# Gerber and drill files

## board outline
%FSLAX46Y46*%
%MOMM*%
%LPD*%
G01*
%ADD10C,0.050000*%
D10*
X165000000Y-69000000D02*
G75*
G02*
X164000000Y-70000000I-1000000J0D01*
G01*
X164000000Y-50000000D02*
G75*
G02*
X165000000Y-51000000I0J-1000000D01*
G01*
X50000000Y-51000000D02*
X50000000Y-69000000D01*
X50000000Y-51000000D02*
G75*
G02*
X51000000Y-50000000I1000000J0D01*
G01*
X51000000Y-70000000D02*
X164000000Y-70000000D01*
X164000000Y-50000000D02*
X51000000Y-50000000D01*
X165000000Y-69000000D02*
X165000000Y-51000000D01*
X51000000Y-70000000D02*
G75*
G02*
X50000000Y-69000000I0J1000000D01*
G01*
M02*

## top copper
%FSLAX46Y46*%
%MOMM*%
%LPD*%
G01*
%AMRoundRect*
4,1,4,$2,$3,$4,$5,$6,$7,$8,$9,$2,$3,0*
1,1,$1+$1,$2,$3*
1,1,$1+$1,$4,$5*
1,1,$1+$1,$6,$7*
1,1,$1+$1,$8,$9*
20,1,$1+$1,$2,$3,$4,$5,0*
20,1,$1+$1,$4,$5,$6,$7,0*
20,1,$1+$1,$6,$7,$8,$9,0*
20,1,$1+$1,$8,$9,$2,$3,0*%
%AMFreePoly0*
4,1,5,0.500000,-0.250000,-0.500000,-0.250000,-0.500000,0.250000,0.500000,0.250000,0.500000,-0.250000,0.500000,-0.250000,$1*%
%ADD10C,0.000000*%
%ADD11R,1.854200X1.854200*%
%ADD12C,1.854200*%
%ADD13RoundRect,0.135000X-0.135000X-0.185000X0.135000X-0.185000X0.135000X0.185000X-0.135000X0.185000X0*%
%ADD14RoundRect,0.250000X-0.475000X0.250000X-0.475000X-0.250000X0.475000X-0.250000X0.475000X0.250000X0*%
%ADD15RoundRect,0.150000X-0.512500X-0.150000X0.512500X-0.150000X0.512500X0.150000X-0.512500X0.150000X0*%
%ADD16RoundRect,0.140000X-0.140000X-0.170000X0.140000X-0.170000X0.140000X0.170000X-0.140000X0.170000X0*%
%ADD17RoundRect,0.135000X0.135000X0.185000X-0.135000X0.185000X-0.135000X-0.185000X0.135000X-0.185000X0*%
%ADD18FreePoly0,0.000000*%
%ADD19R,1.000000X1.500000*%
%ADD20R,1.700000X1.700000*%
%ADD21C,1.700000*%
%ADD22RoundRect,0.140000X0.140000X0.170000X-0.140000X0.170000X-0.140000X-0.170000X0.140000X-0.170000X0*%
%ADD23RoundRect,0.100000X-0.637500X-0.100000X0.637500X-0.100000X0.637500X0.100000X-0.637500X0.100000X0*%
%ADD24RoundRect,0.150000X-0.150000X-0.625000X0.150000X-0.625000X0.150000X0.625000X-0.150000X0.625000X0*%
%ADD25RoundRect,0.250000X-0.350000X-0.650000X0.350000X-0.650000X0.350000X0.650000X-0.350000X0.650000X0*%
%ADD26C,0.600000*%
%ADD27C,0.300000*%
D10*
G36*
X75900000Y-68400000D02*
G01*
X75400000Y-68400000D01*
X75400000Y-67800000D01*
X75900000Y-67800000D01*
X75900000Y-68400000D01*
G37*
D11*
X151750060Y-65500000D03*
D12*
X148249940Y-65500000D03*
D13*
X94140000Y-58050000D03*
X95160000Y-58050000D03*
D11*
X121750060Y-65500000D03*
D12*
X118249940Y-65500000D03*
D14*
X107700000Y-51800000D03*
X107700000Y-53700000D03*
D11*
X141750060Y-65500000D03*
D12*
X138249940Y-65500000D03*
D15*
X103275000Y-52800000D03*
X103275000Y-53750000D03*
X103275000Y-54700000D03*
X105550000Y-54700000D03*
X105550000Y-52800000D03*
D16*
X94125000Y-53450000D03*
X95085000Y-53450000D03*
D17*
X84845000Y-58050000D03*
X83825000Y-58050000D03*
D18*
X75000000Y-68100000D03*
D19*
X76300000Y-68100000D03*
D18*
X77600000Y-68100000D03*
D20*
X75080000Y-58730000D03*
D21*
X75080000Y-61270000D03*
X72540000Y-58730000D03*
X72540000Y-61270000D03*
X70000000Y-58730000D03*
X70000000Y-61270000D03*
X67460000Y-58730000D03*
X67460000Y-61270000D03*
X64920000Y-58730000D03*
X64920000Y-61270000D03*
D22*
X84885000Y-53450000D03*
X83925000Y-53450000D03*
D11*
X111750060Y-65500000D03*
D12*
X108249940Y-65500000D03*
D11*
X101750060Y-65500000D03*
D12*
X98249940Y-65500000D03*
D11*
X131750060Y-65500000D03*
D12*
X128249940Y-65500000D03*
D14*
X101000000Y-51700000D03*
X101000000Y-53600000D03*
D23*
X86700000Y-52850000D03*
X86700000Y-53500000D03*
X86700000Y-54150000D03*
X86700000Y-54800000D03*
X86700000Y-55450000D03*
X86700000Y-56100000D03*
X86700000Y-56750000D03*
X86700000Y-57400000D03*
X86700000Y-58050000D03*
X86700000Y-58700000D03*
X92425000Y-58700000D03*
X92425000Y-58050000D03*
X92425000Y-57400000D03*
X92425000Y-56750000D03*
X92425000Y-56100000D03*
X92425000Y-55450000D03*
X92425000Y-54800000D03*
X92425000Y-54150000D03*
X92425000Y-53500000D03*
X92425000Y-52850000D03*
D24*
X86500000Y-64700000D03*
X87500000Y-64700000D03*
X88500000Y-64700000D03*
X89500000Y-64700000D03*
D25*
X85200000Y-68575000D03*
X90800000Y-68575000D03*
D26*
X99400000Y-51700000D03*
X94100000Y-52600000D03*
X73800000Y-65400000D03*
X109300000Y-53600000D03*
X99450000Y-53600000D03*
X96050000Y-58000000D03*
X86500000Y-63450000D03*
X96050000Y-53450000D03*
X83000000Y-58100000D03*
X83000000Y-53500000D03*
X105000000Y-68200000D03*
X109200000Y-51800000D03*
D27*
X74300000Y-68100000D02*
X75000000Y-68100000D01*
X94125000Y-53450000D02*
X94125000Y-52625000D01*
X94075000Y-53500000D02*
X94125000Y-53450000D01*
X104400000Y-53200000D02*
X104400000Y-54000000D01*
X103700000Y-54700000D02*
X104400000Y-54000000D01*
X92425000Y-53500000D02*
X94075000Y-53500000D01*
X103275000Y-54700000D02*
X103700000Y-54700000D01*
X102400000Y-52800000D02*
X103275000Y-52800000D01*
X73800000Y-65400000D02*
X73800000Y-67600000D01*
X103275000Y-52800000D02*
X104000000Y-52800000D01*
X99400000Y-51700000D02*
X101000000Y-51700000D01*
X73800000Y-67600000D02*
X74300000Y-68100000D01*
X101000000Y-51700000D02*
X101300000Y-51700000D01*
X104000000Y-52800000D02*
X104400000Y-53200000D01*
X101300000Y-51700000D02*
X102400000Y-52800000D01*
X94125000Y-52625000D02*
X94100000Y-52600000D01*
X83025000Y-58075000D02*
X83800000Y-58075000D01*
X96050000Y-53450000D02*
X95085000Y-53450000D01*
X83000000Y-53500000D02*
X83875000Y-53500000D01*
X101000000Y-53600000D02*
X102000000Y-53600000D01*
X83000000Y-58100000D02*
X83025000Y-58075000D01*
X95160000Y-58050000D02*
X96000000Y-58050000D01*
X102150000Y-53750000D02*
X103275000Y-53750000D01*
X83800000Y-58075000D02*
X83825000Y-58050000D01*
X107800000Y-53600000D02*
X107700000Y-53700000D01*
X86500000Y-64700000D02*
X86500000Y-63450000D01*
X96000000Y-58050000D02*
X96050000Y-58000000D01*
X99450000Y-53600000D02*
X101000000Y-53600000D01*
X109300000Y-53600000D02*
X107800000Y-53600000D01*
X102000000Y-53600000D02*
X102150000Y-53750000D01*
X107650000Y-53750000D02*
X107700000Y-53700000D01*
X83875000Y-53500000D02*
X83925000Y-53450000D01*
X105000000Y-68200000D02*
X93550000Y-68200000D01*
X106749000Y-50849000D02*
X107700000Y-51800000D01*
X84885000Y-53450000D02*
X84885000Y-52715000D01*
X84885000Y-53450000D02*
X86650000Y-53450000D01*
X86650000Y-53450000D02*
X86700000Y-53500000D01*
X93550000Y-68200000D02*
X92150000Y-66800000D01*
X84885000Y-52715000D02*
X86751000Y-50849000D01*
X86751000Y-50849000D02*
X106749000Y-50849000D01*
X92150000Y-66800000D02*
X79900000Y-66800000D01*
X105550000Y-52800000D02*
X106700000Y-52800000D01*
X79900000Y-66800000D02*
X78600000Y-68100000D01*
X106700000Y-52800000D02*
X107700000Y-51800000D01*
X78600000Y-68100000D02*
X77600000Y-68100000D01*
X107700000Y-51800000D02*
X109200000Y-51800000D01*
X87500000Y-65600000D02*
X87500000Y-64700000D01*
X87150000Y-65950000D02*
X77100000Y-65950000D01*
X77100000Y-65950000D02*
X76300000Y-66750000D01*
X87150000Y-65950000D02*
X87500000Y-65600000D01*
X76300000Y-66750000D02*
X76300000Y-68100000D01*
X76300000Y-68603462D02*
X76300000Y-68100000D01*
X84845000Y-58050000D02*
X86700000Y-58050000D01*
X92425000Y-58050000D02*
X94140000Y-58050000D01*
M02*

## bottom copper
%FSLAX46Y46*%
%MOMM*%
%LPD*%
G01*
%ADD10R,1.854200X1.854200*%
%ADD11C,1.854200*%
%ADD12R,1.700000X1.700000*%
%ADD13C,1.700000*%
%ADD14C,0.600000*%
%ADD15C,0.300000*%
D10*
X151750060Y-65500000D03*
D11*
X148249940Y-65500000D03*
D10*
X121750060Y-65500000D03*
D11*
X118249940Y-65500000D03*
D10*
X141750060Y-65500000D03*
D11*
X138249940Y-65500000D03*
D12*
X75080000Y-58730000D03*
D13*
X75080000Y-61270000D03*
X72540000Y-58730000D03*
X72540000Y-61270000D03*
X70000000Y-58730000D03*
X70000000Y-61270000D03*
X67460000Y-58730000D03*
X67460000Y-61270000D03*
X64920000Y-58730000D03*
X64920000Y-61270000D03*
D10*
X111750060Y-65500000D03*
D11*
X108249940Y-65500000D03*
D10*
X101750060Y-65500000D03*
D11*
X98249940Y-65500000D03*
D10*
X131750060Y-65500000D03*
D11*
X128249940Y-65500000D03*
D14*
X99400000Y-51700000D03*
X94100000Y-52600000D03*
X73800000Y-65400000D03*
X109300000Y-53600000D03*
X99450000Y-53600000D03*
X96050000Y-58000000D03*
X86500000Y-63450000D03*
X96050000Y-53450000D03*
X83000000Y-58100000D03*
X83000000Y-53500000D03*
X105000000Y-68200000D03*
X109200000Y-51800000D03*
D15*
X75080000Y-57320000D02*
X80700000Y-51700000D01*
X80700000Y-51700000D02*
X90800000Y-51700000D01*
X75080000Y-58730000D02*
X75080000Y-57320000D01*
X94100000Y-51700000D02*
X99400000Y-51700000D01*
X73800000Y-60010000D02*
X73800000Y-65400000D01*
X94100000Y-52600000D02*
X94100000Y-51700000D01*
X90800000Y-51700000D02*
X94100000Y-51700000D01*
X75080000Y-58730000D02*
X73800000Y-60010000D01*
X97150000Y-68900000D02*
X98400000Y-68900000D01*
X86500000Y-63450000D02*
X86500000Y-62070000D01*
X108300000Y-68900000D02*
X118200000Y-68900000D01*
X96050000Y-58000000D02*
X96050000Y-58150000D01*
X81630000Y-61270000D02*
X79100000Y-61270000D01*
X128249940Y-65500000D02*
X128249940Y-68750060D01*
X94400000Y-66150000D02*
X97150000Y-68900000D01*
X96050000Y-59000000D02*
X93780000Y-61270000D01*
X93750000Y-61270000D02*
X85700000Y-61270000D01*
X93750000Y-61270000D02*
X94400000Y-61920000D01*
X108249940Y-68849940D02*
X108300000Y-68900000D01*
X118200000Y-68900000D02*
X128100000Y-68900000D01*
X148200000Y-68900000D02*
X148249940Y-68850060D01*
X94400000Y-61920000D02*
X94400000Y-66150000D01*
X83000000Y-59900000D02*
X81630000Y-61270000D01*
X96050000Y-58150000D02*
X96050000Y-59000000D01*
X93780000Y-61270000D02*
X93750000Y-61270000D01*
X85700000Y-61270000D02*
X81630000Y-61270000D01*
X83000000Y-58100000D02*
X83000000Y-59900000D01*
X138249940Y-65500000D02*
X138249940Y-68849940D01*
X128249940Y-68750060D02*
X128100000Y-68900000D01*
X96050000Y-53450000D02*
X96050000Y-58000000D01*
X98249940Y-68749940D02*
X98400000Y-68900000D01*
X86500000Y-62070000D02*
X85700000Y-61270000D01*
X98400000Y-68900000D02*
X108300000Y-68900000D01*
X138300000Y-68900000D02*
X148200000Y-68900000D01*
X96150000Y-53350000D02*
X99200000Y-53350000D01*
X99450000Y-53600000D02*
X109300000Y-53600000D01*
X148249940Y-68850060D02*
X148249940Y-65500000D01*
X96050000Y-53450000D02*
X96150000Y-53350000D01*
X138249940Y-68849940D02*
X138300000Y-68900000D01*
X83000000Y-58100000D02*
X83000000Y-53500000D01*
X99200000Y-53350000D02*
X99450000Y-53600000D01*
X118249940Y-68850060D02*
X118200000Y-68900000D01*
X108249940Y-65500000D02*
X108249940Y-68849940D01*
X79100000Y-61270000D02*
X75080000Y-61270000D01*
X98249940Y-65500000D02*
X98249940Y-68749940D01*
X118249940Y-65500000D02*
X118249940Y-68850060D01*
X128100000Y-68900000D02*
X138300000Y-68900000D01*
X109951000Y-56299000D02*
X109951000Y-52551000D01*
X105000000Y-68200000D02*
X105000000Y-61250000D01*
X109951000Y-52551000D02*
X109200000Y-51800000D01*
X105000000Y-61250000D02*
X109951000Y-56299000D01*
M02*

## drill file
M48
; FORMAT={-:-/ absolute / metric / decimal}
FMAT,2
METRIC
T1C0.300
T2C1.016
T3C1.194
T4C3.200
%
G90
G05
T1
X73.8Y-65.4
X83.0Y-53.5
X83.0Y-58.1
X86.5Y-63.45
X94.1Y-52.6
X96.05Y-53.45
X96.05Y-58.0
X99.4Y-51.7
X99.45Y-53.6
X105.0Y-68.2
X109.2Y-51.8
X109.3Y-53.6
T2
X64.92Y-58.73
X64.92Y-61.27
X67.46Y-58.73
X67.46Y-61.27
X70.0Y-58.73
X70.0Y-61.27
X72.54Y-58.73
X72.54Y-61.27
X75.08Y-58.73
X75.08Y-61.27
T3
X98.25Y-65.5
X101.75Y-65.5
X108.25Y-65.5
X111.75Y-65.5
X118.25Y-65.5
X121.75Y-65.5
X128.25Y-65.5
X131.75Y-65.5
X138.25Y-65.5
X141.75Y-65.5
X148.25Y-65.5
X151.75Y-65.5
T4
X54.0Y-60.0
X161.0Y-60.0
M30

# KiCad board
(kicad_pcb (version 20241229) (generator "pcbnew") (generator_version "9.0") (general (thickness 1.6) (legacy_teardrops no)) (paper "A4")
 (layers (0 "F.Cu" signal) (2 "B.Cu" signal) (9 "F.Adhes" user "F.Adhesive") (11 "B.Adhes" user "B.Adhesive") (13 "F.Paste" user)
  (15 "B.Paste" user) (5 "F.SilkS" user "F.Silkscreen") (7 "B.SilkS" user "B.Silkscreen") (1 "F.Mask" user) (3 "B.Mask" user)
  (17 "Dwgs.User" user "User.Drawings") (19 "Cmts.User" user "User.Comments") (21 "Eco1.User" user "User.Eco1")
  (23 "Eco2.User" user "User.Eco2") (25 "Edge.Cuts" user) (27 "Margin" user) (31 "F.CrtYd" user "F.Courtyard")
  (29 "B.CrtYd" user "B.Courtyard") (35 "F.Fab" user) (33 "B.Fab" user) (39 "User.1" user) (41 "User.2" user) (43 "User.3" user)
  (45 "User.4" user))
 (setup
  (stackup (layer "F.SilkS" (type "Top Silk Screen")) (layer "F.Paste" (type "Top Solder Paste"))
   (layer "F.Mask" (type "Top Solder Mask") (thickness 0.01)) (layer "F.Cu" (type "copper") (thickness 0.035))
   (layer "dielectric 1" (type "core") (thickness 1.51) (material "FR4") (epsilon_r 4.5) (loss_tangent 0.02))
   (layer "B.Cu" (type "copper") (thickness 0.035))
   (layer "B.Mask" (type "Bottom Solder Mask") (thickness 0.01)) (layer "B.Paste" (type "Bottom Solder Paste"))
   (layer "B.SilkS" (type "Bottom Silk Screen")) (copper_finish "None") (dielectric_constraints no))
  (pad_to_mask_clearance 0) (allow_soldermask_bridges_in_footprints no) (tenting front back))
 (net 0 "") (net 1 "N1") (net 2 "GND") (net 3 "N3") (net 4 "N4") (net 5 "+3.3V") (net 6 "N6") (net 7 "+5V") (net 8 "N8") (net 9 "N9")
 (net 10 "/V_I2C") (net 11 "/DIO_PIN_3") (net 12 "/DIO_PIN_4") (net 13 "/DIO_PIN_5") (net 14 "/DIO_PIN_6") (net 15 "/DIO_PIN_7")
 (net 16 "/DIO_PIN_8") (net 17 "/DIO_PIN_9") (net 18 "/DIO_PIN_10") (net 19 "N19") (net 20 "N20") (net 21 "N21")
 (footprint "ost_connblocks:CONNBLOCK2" (layer "F.Cu") (at 150 65.5 180)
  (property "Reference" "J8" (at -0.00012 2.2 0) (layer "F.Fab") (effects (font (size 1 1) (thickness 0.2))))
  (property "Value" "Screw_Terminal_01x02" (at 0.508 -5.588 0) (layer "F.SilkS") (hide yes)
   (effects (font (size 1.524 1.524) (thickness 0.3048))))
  (pad "1" thru_hole rect (at -1.75006 0 180) (size 1.8542 1.8542) (drill 1.1938) (layers "*.Cu" "*.Mask") (remove_unused_layers no)
   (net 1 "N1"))
  (pad "2" thru_hole circle (at 1.75006 0 180) (size 1.8542 1.8542) (drill 1.1938) (layers "*.Cu" "*.Mask") (remove_unused_layers no)
   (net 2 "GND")))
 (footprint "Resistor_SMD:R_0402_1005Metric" (layer "F.Cu") (at 94.65 58.05)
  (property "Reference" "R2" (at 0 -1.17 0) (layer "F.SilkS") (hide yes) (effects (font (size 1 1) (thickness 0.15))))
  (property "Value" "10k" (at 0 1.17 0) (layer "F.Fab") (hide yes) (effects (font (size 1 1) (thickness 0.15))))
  (pad "1" smd roundrect (at -0.51 0) (size 0.54 0.64) (layers "F.Cu" "F.Mask" "F.Paste") (roundrect_rratio 0.25) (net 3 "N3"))
  (pad "2" smd roundrect (at 0.51 0) (size 0.54 0.64) (layers "F.Cu" "F.Mask" "F.Paste") (roundrect_rratio 0.25) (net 2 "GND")))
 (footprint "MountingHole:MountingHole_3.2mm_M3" (layer "F.Cu") (at 54 60)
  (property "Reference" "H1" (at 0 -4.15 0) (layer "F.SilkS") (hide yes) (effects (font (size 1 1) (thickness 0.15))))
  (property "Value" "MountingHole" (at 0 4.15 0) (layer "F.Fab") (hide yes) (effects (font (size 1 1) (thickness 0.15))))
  (pad "" np_thru_hole circle (at 0 0) (size 3.2 3.2) (drill 3.2) (layers "*.Cu" "*.Mask")))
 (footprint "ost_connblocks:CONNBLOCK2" (layer "F.Cu") (at 120 65.5 180)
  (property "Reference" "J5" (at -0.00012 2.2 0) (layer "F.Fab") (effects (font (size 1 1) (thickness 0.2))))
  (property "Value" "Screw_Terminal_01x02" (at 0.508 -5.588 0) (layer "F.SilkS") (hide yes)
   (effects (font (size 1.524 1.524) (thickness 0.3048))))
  (pad "1" thru_hole rect (at -1.75006 0 180) (size 1.8542 1.8542) (drill 1.1938) (layers "*.Cu" "*.Mask") (remove_unused_layers no)
   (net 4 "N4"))
  (pad "2" thru_hole circle (at 1.75006 0 180) (size 1.8542 1.8542) (drill 1.1938) (layers "*.Cu" "*.Mask") (remove_unused_layers no)
   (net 2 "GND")))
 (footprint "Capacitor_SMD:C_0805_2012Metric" (layer "F.Cu") (at 107.7 52.75 -90)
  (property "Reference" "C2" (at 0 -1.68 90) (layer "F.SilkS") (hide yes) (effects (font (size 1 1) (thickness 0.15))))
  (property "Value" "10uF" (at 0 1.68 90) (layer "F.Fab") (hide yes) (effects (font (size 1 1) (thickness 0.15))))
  (pad "1" smd roundrect (at -0.95 0 270) (size 1 1.45) (layers "F.Cu" "F.Mask" "F.Paste") (roundrect_rratio 0.25) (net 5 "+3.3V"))
  (pad "2" smd roundrect (at 0.95 0 270) (size 1 1.45) (layers "F.Cu" "F.Mask" "F.Paste") (roundrect_rratio 0.25) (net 2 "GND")))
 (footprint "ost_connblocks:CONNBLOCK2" (layer "F.Cu") (at 140 65.5 180)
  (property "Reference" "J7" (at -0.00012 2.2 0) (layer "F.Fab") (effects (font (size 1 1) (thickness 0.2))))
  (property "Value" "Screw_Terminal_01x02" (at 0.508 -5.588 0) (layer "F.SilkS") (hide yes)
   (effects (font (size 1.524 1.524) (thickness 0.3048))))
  (pad "1" thru_hole rect (at -1.75006 0 180) (size 1.8542 1.8542) (drill 1.1938) (layers "*.Cu" "*.Mask") (remove_unused_layers no)
   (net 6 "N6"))
  (pad "2" thru_hole circle (at 1.75006 0 180) (size 1.8542 1.8542) (drill 1.1938) (layers "*.Cu" "*.Mask") (remove_unused_layers no)
   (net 2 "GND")))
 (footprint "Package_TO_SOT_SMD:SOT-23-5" (layer "F.Cu") (at 104.4125 53.75)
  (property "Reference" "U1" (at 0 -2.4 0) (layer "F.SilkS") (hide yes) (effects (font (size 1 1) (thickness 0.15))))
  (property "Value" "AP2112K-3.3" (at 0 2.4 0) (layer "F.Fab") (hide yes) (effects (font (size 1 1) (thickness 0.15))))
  (pad "1" smd roundrect (at -1.1375 -0.95) (size 1.325 0.6) (layers "F.Cu" "F.Mask" "F.Paste") (roundrect_rratio 0.25) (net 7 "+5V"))
  (pad "2" smd roundrect (at -1.1375 0) (size 1.325 0.6) (layers "F.Cu" "F.Mask" "F.Paste") (roundrect_rratio 0.25) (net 2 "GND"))
  (pad "3" smd roundrect (at -1.1375 0.95) (size 1.325 0.6) (layers "F.Cu" "F.Mask" "F.Paste") (roundrect_rratio 0.25) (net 7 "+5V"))
  (pad "4" smd roundrect (at 1.1375 0.95) (size 1.325 0.6) (layers "F.Cu" "F.Mask" "F.Paste") (roundrect_rratio 0.25) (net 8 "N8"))
  (pad "5" smd roundrect (at 1.1375 -0.95) (size 1.325 0.6) (layers "F.Cu" "F.Mask" "F.Paste") (roundrect_rratio 0.25) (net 5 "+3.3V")))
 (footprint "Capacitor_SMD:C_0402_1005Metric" (layer "F.Cu") (at 94.605 53.45)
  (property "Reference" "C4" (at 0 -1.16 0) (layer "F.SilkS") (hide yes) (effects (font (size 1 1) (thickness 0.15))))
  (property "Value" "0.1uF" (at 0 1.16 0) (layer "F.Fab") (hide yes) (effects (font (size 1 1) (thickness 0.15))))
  (pad "1" smd roundrect (at -0.48 0) (size 0.56 0.62) (layers "F.Cu" "F.Mask" "F.Paste") (roundrect_rratio 0.25) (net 7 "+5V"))
  (pad "2" smd roundrect (at 0.48 0) (size 0.56 0.62) (layers "F.Cu" "F.Mask" "F.Paste") (roundrect_rratio 0.25) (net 2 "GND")))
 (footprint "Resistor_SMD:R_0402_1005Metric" (layer "F.Cu") (at 84.335 58.05 180)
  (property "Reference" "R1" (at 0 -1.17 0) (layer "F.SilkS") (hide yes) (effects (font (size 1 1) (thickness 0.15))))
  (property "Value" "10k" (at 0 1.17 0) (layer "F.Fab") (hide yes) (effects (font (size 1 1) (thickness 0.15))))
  (pad "1" smd roundrect (at -0.51 0 180) (size 0.54 0.64) (layers "F.Cu" "F.Mask" "F.Paste") (roundrect_rratio 0.25) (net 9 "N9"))
  (pad "2" smd roundrect (at 0.51 0 180) (size 0.54 0.64) (layers "F.Cu" "F.Mask" "F.Paste") (roundrect_rratio 0.25) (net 2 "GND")))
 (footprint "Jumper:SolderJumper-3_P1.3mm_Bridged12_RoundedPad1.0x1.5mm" (layer "F.Cu") (at 76.3 68.1)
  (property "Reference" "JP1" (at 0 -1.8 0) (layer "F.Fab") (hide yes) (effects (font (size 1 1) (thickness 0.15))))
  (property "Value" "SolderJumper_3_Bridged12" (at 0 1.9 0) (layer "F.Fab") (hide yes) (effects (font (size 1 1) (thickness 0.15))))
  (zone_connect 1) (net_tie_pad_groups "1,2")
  (fp_poly (pts (xy -0.9 -0.3) (xy -0.4 -0.3) (xy -0.4 0.3) (xy -0.9 0.3)) (stroke (width 0) (type solid)) (fill yes) (layer "F.Cu"))
  (pad "1" smd custom (at -1.3 0) (size 1 0.5) (layers "F.Cu" "F.Mask") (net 7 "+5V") (zone_connect 2) (thermal_bridge_angle 45)
   (options (clearance outline) (anchor rect)) (primitives))
  (pad "2" smd rect (at 0 0) (size 1 1.5) (layers "F.Cu" "F.Mask") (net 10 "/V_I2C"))
  (pad "3" smd custom (at 1.3 0) (size 1 0.5) (layers "F.Cu" "F.Mask") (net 5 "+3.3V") (zone_connect 2) (thermal_bridge_angle 45)
   (options (clearance outline) (anchor rect)) (primitives)))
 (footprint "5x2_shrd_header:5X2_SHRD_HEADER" (layer "F.Cu") (at 70 60 180)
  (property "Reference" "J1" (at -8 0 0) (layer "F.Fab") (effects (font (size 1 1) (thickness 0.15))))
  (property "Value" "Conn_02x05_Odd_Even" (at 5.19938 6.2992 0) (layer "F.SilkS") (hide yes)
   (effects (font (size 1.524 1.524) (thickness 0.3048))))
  (pad "1" thru_hole rect (at -5.08 1.27 180) (size 1.7 1.7) (drill 1.016) (layers "*.Cu" "*.Mask") (remove_unused_layers no) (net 7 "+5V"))
  (pad "2" thru_hole circle (at -5.08 -1.27 180) (size 1.7 1.7) (drill 1.016) (layers "*.Cu" "*.Mask") (remove_unused_layers no)
   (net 2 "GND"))
  (pad "3" thru_hole circle (at -2.54 1.27 180) (size 1.7 1.7) (drill 1.016) (layers "*.Cu" "*.Mask") (remove_unused_layers no)
   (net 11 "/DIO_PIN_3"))
  (pad "4" thru_hole circle (at -2.54 -1.27 180) (size 1.7 1.7) (drill 1.016) (layers "*.Cu" "*.Mask") (remove_unused_layers no)
   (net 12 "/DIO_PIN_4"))
  (pad "5" thru_hole circle (at 0 1.27 180) (size 1.7 1.7) (drill 1.016) (layers "*.Cu" "*.Mask") (remove_unused_layers no)
   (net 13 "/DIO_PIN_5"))
  (pad "6" thru_hole circle (at 0 -1.27 180) (size 1.7 1.7) (drill 1.016) (layers "*.Cu" "*.Mask") (remove_unused_layers no)
   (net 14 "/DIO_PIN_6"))
  (pad "7" thru_hole circle (at 2.54 1.27 180) (size 1.7 1.7) (drill 1.016) (layers "*.Cu" "*.Mask") (remove_unused_layers no)
   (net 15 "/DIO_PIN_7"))
  (pad "8" thru_hole circle (at 2.54 -1.27 180) (size 1.7 1.7) (drill 1.016) (layers "*.Cu" "*.Mask") (remove_unused_layers no)
   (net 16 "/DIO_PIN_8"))
  (pad "9" thru_hole circle (at 5.08 1.27 180) (size 1.7 1.7) (drill 1.016) (layers "*.Cu" "*.Mask") (remove_unused_layers no)
   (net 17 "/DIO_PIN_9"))
  (pad "10" thru_hole circle (at 5.08 -1.27 180) (size 1.7 1.7) (drill 1.016) (layers "*.Cu" "*.Mask") (remove_unused_layers no)
   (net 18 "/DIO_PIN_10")))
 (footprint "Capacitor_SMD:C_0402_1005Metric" (layer "F.Cu") (at 84.405 53.45 180)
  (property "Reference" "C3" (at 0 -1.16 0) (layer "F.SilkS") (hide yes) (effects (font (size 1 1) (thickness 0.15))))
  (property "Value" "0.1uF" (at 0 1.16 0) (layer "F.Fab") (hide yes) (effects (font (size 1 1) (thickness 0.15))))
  (pad "1" smd roundrect (at -0.48 0 180) (size 0.56 0.62) (layers "F.Cu" "F.Mask" "F.Paste") (roundrect_rratio 0.25) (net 5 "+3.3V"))
  (pad "2" smd roundrect (at 0.48 0 180) (size 0.56 0.62) (layers "F.Cu" "F.Mask" "F.Paste") (roundrect_rratio 0.25) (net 2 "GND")))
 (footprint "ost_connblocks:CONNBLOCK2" (layer "F.Cu") (at 110 65.5 180)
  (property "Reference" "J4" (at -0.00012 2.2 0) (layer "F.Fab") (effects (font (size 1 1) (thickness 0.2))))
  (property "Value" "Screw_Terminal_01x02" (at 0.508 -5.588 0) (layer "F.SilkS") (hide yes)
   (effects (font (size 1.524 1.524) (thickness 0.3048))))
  (pad "1" thru_hole rect (at -1.75006 0 180) (size 1.8542 1.8542) (drill 1.1938) (layers "*.Cu" "*.Mask") (remove_unused_layers no)
   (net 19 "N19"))
  (pad "2" thru_hole circle (at 1.75006 0 180) (size 1.8542 1.8542) (drill 1.1938) (layers "*.Cu" "*.Mask") (remove_unused_layers no)
   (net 2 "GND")))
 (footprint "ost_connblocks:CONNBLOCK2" (layer "F.Cu") (at 100 65.5 180)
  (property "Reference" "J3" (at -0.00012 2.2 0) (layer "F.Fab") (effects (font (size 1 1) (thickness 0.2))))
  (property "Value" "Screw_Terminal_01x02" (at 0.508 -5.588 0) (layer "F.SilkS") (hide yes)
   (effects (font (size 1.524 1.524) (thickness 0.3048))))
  (pad "1" thru_hole rect (at -1.75006 0 180) (size 1.8542 1.8542) (drill 1.1938) (layers "*.Cu" "*.Mask") (remove_unused_layers no)
   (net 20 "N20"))
  (pad "2" thru_hole circle (at 1.75006 0 180) (size 1.8542 1.8542) (drill 1.1938) (layers "*.Cu" "*.Mask") (remove_unused_layers no)
   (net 2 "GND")))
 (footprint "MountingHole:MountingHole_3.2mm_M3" (layer "F.Cu") (at 161 60)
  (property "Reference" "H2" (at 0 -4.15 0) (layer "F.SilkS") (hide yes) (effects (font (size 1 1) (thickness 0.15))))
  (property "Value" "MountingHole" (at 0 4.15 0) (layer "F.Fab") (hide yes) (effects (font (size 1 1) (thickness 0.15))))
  (pad "" np_thru_hole circle (at 0 0) (size 3.2 3.2) (drill 3.2) (layers "*.Cu" "*.Mask")))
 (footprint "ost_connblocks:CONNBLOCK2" (layer "F.Cu") (at 130 65.5 180)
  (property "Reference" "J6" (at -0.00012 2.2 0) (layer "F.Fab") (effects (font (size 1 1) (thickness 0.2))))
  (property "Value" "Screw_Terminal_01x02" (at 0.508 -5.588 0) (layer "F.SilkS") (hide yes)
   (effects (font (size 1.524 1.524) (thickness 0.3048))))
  (pad "1" thru_hole rect (at -1.75006 0 180) (size 1.8542 1.8542) (drill 1.1938) (layers "*.Cu" "*.Mask") (remove_unused_layers no)
   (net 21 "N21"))
  (pad "2" thru_hole circle (at 1.75006 0 180) (size 1.8542 1.8542) (drill 1.1938) (layers "*.Cu" "*.Mask") (remove_unused_layers no)
   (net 2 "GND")))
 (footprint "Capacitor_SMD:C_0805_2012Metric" (layer "F.Cu") (at 101 52.65 -90)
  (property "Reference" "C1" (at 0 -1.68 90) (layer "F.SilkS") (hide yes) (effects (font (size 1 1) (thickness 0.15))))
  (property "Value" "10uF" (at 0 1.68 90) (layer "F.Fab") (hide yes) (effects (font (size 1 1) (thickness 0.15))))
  (pad "1" smd roundrect (at -0.95 0 270) (size 1 1.45) (layers "F.Cu" "F.Mask" "F.Paste") (roundrect_rratio 0.25) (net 7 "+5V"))
  (pad "2" smd roundrect (at 0.95 0 270) (size 1 1.45) (layers "F.Cu" "F.Mask" "F.Paste") (roundrect_rratio 0.25) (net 2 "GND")))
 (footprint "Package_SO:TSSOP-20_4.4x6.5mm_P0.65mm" (layer "F.Cu") (at 89.5625 55.775)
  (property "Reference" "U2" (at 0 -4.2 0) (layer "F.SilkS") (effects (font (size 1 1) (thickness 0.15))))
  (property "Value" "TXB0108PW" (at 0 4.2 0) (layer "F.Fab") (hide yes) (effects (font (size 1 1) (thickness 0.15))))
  (pad "1" smd roundrect (at -2.8625 -2.925) (size 1.475 0.4) (layers "F.Cu" "F.Mask" "F.Paste") (roundrect_rratio 0.25)
   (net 11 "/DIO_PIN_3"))
  (pad "2" smd roundrect (at -2.8625 -2.275) (size 1.475 0.4) (layers "F.Cu" "F.Mask" "F.Paste") (roundrect_rratio 0.25) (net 5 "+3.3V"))
  (pad "3" smd roundrect (at -2.8625 -1.625) (size 1.475 0.4) (layers "F.Cu" "F.Mask" "F.Paste") (roundrect_rratio 0.25)
   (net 12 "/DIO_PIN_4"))
  (pad "4" smd roundrect (at -2.8625 -0.975) (size 1.475 0.4) (layers "F.Cu" "F.Mask" "F.Paste") (roundrect_rratio 0.25)
   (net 15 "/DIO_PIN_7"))
  (pad "5" smd roundrect (at -2.8625 -0.325) (size 1.475 0.4) (layers "F.Cu" "F.Mask" "F.Paste") (roundrect_rratio 0.25)
   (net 16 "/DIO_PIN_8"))
  (pad "6" smd roundrect (at -2.8625 0.325) (size 1.475 0.4) (layers "F.Cu" "F.Mask" "F.Paste") (roundrect_rratio 0.25)
   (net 17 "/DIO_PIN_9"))
  (pad "7" smd roundrect (at -2.8625 0.975) (size 1.475 0.4) (layers "F.Cu" "F.Mask" "F.Paste") (roundrect_rratio 0.25)
   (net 18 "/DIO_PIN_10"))
  (pad "8" smd roundrect (at -2.8625 1.625) (size 1.475 0.4) (layers "F.Cu" "F.Mask" "F.Paste") (roundrect_rratio 0.25) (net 9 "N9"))
  (pad "9" smd roundrect (at -2.8625 2.275) (size 1.475 0.4) (layers "F.Cu" "F.Mask" "F.Paste") (roundrect_rratio 0.25) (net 9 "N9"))
  (pad "10" smd roundrect (at -2.8625 2.925) (size 1.475 0.4) (layers "F.Cu" "F.Mask" "F.Paste") (roundrect_rratio 0.25) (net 5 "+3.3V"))
  (pad "11" smd roundrect (at 2.8625 2.925) (size 1.475 0.4) (layers "F.Cu" "F.Mask" "F.Paste") (roundrect_rratio 0.25) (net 2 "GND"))
  (pad "12" smd roundrect (at 2.8625 2.275) (size 1.475 0.4) (layers "F.Cu" "F.Mask" "F.Paste") (roundrect_rratio 0.25) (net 3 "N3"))
  (pad "13" smd roundrect (at 2.8625 1.625) (size 1.475 0.4) (layers "F.Cu" "F.Mask" "F.Paste") (roundrect_rratio 0.25) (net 3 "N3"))
  (pad "14" smd roundrect (at 2.8625 0.975) (size 1.475 0.4) (layers "F.Cu" "F.Mask" "F.Paste") (roundrect_rratio 0.25) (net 1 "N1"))
  (pad "15" smd roundrect (at 2.8625 0.325) (size 1.475 0.4) (layers "F.Cu" "F.Mask" "F.Paste") (roundrect_rratio 0.25) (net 6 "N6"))
  (pad "16" smd roundrect (at 2.8625 -0.325) (size 1.475 0.4) (layers "F.Cu" "F.Mask" "F.Paste") (roundrect_rratio 0.25) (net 21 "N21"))
  (pad "17" smd roundrect (at 2.8625 -0.975) (size 1.475 0.4) (layers "F.Cu" "F.Mask" "F.Paste") (roundrect_rratio 0.25) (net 4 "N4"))
  (pad "18" smd roundrect (at 2.8625 -1.625) (size 1.475 0.4) (layers "F.Cu" "F.Mask" "F.Paste") (roundrect_rratio 0.25) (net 19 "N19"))
  (pad "19" smd roundrect (at 2.8625 -2.275) (size 1.475 0.4) (layers "F.Cu" "F.Mask" "F.Paste") (roundrect_rratio 0.25) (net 7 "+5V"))
  (pad "20" smd roundrect (at 2.8625 -2.925) (size 1.475 0.4) (layers "F.Cu" "F.Mask" "F.Paste") (roundrect_rratio 0.25) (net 20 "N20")))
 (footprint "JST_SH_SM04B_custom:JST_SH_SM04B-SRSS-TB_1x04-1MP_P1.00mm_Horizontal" (layer "F.Cu") (at 88 66.7)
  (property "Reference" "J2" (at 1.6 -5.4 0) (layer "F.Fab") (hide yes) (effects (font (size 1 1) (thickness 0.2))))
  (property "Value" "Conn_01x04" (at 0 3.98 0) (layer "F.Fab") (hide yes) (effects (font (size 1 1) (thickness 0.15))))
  (pad "1" smd roundrect (at -1.5 -2) (size 0.6 1.55) (layers "F.Cu" "F.Mask" "F.Paste") (roundrect_rratio 0.25) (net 2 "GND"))
  (pad "2" smd roundrect (at -0.5 -2) (size 0.6 1.55) (layers "F.Cu" "F.Mask" "F.Paste") (roundrect_rratio 0.25) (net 10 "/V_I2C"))
  (pad "3" smd roundrect (at 0.5 -2) (size 0.6 1.55) (layers "F.Cu" "F.Mask" "F.Paste") (roundrect_rratio 0.25) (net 14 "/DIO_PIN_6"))
  (pad "4" smd roundrect (at 1.5 -2) (size 0.6 1.55) (layers "F.Cu" "F.Mask" "F.Paste") (roundrect_rratio 0.25) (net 13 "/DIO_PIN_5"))
  (pad "MP" smd roundrect (at -2.8 1.875) (size 1.2 1.8) (layers "F.Cu" "F.Mask" "F.Paste") (roundrect_rratio 0.208333))
  (pad "MP" smd roundrect (at 2.8 1.875) (size 1.2 1.8) (layers "F.Cu" "F.Mask" "F.Paste") (roundrect_rratio 0.208333)))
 (gr_arc (start 165 69) (mid 164.707107 69.707107) (end 164 70) (stroke (width 0.05) (type default)) (layer "Edge.Cuts"))
 (gr_arc (start 164 50) (mid 164.707107 50.292893) (end 165 51) (stroke (width 0.05) (type default)) (layer "Edge.Cuts"))
 (gr_line (start 50 51) (end 50 69) (stroke (width 0.05) (type default)) (layer "Edge.Cuts"))
 (gr_arc (start 50 51) (mid 50.292893 50.292893) (end 51 50) (stroke (width 0.05) (type default)) (layer "Edge.Cuts"))
 (gr_line (start 51 70) (end 164 70) (stroke (width 0.05) (type default)) (layer "Edge.Cuts"))
 (gr_line (start 164 50) (end 51 50) (stroke (width 0.05) (type default)) (layer "Edge.Cuts"))
 (gr_line (start 165 69) (end 165 51) (stroke (width 0.05) (type default)) (layer "Edge.Cuts"))
 (gr_arc (start 51 70) (mid 50.292893 69.707107) (end 50 69) (stroke (width 0.05) (type default)) (layer "Edge.Cuts"))
 (segment (start 74.3 68.1) (end 75 68.1) (width 0.3) (layer "F.Cu") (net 7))
 (segment (start 94.125 53.45) (end 94.125 52.625) (width 0.3) (layer "F.Cu") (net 7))
 (segment (start 94.075 53.5) (end 94.125 53.45) (width 0.3) (layer "F.Cu") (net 7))
 (segment (start 104.4 53.2) (end 104.4 54) (width 0.3) (layer "F.Cu") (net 7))
 (segment (start 103.7 54.7) (end 104.4 54) (width 0.3) (layer "F.Cu") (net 7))
 (segment (start 92.425 53.5) (end 94.075 53.5) (width 0.3) (layer "F.Cu") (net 7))
 (segment (start 103.275 54.7) (end 103.7 54.7) (width 0.3) (layer "F.Cu") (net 7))
 (segment (start 102.4 52.8) (end 103.275 52.8) (width 0.3) (layer "F.Cu") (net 7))
 (segment (start 73.8 65.4) (end 73.8 67.6) (width 0.3) (layer "F.Cu") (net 7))
 (segment (start 103.275 52.8) (end 104 52.8) (width 0.3) (layer "F.Cu") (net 7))
 (segment (start 99.4 51.7) (end 101 51.7) (width 0.3) (layer "F.Cu") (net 7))
 (segment (start 73.8 67.6) (end 74.3 68.1) (width 0.3) (layer "F.Cu") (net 7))
 (segment (start 101 51.7) (end 101.3 51.7) (width 0.3) (layer "F.Cu") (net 7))
 (segment (start 104 52.8) (end 104.4 53.2) (width 0.3) (layer "F.Cu") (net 7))
 (segment (start 101.3 51.7) (end 102.4 52.8) (width 0.3) (layer "F.Cu") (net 7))
 (segment (start 94.125 52.625) (end 94.1 52.6) (width 0.3) (layer "F.Cu") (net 7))
 (via (at 99.4 51.7) (size 0.6) (drill 0.3) (layers "F.Cu" "B.Cu") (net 7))
 (via (at 94.1 52.6) (size 0.6) (drill 0.3) (layers "F.Cu" "B.Cu") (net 7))
 (via (at 73.8 65.4) (size 0.6) (drill 0.3) (layers "F.Cu" "B.Cu") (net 7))
 (segment (start 75.08 57.32) (end 80.7 51.7) (width 0.3) (layer "B.Cu") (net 7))
 (segment (start 80.7 51.7) (end 90.8 51.7) (width 0.3) (layer "B.Cu") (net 7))
 (segment (start 75.08 58.73) (end 75.08 57.32) (width 0.3) (layer "B.Cu") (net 7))
 (segment (start 94.1 51.7) (end 99.4 51.7) (width 0.3) (layer "B.Cu") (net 7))
 (segment (start 73.8 60.01) (end 73.8 65.4) (width 0.3) (layer "B.Cu") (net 7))
 (segment (start 94.1 52.6) (end 94.1 51.7) (width 0.3) (layer "B.Cu") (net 7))
 (segment (start 90.8 51.7) (end 94.1 51.7) (width 0.3) (layer "B.Cu") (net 7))
 (segment (start 75.08 58.73) (end 73.8 60.01) (width 0.3) (layer "B.Cu") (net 7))
 (segment (start 83.025 58.075) (end 83.8 58.075) (width 0.3) (layer "F.Cu") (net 2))
 (segment (start 96.05 53.45) (end 95.085 53.45) (width 0.3) (layer "F.Cu") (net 2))
 (segment (start 83 53.5) (end 83.875 53.5) (width 0.3) (layer "F.Cu") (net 2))
 (segment (start 101 53.6) (end 102 53.6) (width 0.3) (layer "F.Cu") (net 2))
 (segment (start 83 58.1) (end 83.025 58.075) (width 0.3) (layer "F.Cu") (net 2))
 (segment (start 95.16 58.05) (end 96 58.05) (width 0.3) (layer "F.Cu") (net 2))
 (segment (start 102.15 53.75) (end 103.275 53.75) (width 0.3) (layer "F.Cu") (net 2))
 (segment (start 83.8 58.075) (end 83.825 58.05) (width 0.3) (layer "F.Cu") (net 2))
 (segment (start 107.8 53.6) (end 107.7 53.7) (width 0.3) (layer "F.Cu") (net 2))
 (segment (start 86.5 64.7) (end 86.5 63.45) (width 0.3) (layer "F.Cu") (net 2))
 (segment (start 96 58.05) (end 96.05 58) (width 0.3) (layer "F.Cu") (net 2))
 (segment (start 99.45 53.6) (end 101 53.6) (width 0.3) (layer "F.Cu") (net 2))
 (segment (start 109.3 53.6) (end 107.8 53.6) (width 0.3) (layer "F.Cu") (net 2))
 (segment (start 102 53.6) (end 102.15 53.75) (width 0.3) (layer "F.Cu") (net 2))
 (segment (start 107.65 53.75) (end 107.7 53.7) (width 0.3) (layer "F.Cu") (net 2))
 (segment (start 83.875 53.5) (end 83.925 53.45) (width 0.3) (layer "F.Cu") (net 2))
 (via (at 109.3 53.6) (size 0.6) (drill 0.3) (layers "F.Cu" "B.Cu") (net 2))
 (via (at 99.45 53.6) (size 0.6) (drill 0.3) (layers "F.Cu" "B.Cu") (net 2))
 (via (at 96.05 58) (size 0.6) (drill 0.3) (layers "F.Cu" "B.Cu") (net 2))
 (via (at 86.5 63.45) (size 0.6) (drill 0.3) (layers "F.Cu" "B.Cu") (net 2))
 (via (at 96.05 53.45) (size 0.6) (drill 0.3) (layers "F.Cu" "B.Cu") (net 2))
 (via (at 83 58.1) (size 0.6) (drill 0.3) (layers "F.Cu" "B.Cu") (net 2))
 (via (at 83 53.5) (size 0.6) (drill 0.3) (layers "F.Cu" "B.Cu") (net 2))
 (segment (start 97.15 68.9) (end 98.4 68.9) (width 0.3) (layer "B.Cu") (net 2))
 (segment (start 86.5 63.45) (end 86.5 62.07) (width 0.3) (layer "B.Cu") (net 2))
 (segment (start 108.3 68.9) (end 118.2 68.9) (width 0.3) (layer "B.Cu") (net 2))
 (segment (start 96.05 58) (end 96.05 58.15) (width 0.3) (layer "B.Cu") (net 2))
 (segment (start 81.63 61.27) (end 79.1 61.27) (width 0.3) (layer "B.Cu") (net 2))
 (segment (start 128.24994 65.5) (end 128.24994 68.75006) (width 0.3) (layer "B.Cu") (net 2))
 (segment (start 94.4 66.15) (end 97.15 68.9) (width 0.3) (layer "B.Cu") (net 2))
 (segment (start 96.05 59) (end 93.78 61.27) (width 0.3) (layer "B.Cu") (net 2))
 (segment (start 93.75 61.27) (end 85.7 61.27) (width 0.3) (layer "B.Cu") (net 2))
 (segment (start 93.75 61.27) (end 94.4 61.92) (width 0.3) (layer "B.Cu") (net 2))
 (segment (start 108.24994 68.84994) (end 108.3 68.9) (width 0.3) (layer "B.Cu") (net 2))
 (segment (start 118.2 68.9) (end 128.1 68.9) (width 0.3) (layer "B.Cu") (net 2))
 (segment (start 148.2 68.9) (end 148.24994 68.85006) (width 0.3) (layer "B.Cu") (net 2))
 (segment (start 94.4 61.92) (end 94.4 66.15) (width 0.3) (layer "B.Cu") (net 2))
 (segment (start 83 59.9) (end 81.63 61.27) (width 0.3) (layer "B.Cu") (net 2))
 (segment (start 96.05 58.15) (end 96.05 59) (width 0.3) (layer "B.Cu") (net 2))
 (segment (start 93.78 61.27) (end 93.75 61.27) (width 0.3) (layer "B.Cu") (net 2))
 (segment (start 85.7 61.27) (end 81.63 61.27) (width 0.3) (layer "B.Cu") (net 2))
 (segment (start 83 58.1) (end 83 59.9) (width 0.3) (layer "B.Cu") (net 2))
 (segment (start 138.24994 65.5) (end 138.24994 68.84994) (width 0.3) (layer "B.Cu") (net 2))
 (segment (start 128.24994 68.75006) (end 128.1 68.9) (width 0.3) (layer "B.Cu") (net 2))
 (segment (start 96.05 53.45) (end 96.05 58) (width 0.3) (layer "B.Cu") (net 2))
 (segment (start 98.24994 68.74994) (end 98.4 68.9) (width 0.3) (layer "B.Cu") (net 2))
 (segment (start 86.5 62.07) (end 85.7 61.27) (width 0.3) (layer "B.Cu") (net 2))
 (segment (start 98.4 68.9) (end 108.3 68.9) (width 0.3) (layer "B.Cu") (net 2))
 (segment (start 138.3 68.9) (end 148.2 68.9) (width 0.3) (layer "B.Cu") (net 2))
 (segment (start 96.15 53.35) (end 99.2 53.35) (width 0.3) (layer "B.Cu") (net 2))
 (segment (start 99.45 53.6) (end 109.3 53.6) (width 0.3) (layer "B.Cu") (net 2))
 (segment (start 148.24994 68.85006) (end 148.24994 65.5) (width 0.3) (layer "B.Cu") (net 2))
 (segment (start 96.05 53.45) (end 96.15 53.35) (width 0.3) (layer "B.Cu") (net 2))
 (segment (start 138.24994 68.84994) (end 138.3 68.9) (width 0.3) (layer "B.Cu") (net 2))
 (segment (start 83 58.1) (end 83 53.5) (width 0.3) (layer "B.Cu") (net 2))
 (segment (start 99.2 53.35) (end 99.45 53.6) (width 0.3) (layer "B.Cu") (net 2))
 (segment (start 118.24994 68.85006) (end 118.2 68.9) (width 0.3) (layer "B.Cu") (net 2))
 (segment (start 108.24994 65.5) (end 108.24994 68.84994) (width 0.3) (layer "B.Cu") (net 2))
 (segment (start 79.1 61.27) (end 75.08 61.27) (width 0.3) (layer "B.Cu") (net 2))
 (segment (start 98.24994 65.5) (end 98.24994 68.74994) (width 0.3) (layer "B.Cu") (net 2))
 (segment (start 118.24994 65.5) (end 118.24994 68.85006) (width 0.3) (layer "B.Cu") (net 2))
 (segment (start 128.1 68.9) (end 138.3 68.9) (width 0.3) (layer "B.Cu") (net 2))
 (segment (start 105 68.2) (end 93.55 68.2) (width 0.3) (layer "F.Cu") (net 5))
 (segment (start 106.749 50.849) (end 107.7 51.8) (width 0.3) (layer "F.Cu") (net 5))
 (segment (start 84.885 53.45) (end 84.885 52.715) (width 0.3) (layer "F.Cu") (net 5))
 (segment (start 84.885 53.45) (end 86.65 53.45) (width 0.3) (layer "F.Cu") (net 5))
 (segment (start 86.65 53.45) (end 86.7 53.5) (width 0.3) (layer "F.Cu") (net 5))
 (segment (start 93.55 68.2) (end 92.15 66.8) (width 0.3) (layer "F.Cu") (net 5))
 (segment (start 84.885 52.715) (end 86.751 50.849) (width 0.3) (layer "F.Cu") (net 5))
 (segment (start 86.751 50.849) (end 106.749 50.849) (width 0.3) (layer "F.Cu") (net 5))
 (segment (start 92.15 66.8) (end 79.9 66.8) (width 0.3) (layer "F.Cu") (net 5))
 (segment (start 105.55 52.8) (end 106.7 52.8) (width 0.3) (layer "F.Cu") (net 5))
 (segment (start 79.9 66.8) (end 78.6 68.1) (width 0.3) (layer "F.Cu") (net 5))
 (segment (start 106.7 52.8) (end 107.7 51.8) (width 0.3) (layer "F.Cu") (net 5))
 (segment (start 78.6 68.1) (end 77.6 68.1) (width 0.3) (layer "F.Cu") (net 5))
 (segment (start 107.7 51.8) (end 109.2 51.8) (width 0.3) (layer "F.Cu") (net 5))
 (via (at 105 68.2) (size 0.6) (drill 0.3) (layers "F.Cu" "B.Cu") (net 5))
 (via (at 109.2 51.8) (size 0.6) (drill 0.3) (layers "F.Cu" "B.Cu") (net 5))
 (segment (start 109.951 56.299) (end 109.951 52.551) (width 0.3) (layer "B.Cu") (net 5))
 (segment (start 105 68.2) (end 105 61.25) (width 0.3) (layer "B.Cu") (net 5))
 (segment (start 109.951 52.551) (end 109.2 51.8) (width 0.3) (layer "B.Cu") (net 5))
 (segment (start 105 61.25) (end 109.951 56.299) (width 0.3) (layer "B.Cu") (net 5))
 (segment (start 87.5 65.6) (end 87.5 64.7) (width 0.3) (layer "F.Cu") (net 10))
 (segment (start 87.15 65.95) (end 77.1 65.95) (width 0.3) (layer "F.Cu") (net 10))
 (segment (start 77.1 65.95) (end 76.3 66.75) (width 0.3) (layer "F.Cu") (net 10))
 (segment (start 87.15 65.95) (end 87.5 65.6) (width 0.3) (layer "F.Cu") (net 10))
 (segment (start 76.3 66.75) (end 76.3 68.1) (width 0.3) (layer "F.Cu") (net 10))
 (segment (start 76.3 68.603462) (end 76.3 68.1) (width 0.3) (layer "F.Cu") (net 10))
 (segment (start 84.845 58.05) (end 86.7 58.05) (width 0.3) (layer "F.Cu") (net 9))
 (segment (start 92.425 58.05) (end 94.14 58.05) (width 0.3) (layer "F.Cu") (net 3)))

